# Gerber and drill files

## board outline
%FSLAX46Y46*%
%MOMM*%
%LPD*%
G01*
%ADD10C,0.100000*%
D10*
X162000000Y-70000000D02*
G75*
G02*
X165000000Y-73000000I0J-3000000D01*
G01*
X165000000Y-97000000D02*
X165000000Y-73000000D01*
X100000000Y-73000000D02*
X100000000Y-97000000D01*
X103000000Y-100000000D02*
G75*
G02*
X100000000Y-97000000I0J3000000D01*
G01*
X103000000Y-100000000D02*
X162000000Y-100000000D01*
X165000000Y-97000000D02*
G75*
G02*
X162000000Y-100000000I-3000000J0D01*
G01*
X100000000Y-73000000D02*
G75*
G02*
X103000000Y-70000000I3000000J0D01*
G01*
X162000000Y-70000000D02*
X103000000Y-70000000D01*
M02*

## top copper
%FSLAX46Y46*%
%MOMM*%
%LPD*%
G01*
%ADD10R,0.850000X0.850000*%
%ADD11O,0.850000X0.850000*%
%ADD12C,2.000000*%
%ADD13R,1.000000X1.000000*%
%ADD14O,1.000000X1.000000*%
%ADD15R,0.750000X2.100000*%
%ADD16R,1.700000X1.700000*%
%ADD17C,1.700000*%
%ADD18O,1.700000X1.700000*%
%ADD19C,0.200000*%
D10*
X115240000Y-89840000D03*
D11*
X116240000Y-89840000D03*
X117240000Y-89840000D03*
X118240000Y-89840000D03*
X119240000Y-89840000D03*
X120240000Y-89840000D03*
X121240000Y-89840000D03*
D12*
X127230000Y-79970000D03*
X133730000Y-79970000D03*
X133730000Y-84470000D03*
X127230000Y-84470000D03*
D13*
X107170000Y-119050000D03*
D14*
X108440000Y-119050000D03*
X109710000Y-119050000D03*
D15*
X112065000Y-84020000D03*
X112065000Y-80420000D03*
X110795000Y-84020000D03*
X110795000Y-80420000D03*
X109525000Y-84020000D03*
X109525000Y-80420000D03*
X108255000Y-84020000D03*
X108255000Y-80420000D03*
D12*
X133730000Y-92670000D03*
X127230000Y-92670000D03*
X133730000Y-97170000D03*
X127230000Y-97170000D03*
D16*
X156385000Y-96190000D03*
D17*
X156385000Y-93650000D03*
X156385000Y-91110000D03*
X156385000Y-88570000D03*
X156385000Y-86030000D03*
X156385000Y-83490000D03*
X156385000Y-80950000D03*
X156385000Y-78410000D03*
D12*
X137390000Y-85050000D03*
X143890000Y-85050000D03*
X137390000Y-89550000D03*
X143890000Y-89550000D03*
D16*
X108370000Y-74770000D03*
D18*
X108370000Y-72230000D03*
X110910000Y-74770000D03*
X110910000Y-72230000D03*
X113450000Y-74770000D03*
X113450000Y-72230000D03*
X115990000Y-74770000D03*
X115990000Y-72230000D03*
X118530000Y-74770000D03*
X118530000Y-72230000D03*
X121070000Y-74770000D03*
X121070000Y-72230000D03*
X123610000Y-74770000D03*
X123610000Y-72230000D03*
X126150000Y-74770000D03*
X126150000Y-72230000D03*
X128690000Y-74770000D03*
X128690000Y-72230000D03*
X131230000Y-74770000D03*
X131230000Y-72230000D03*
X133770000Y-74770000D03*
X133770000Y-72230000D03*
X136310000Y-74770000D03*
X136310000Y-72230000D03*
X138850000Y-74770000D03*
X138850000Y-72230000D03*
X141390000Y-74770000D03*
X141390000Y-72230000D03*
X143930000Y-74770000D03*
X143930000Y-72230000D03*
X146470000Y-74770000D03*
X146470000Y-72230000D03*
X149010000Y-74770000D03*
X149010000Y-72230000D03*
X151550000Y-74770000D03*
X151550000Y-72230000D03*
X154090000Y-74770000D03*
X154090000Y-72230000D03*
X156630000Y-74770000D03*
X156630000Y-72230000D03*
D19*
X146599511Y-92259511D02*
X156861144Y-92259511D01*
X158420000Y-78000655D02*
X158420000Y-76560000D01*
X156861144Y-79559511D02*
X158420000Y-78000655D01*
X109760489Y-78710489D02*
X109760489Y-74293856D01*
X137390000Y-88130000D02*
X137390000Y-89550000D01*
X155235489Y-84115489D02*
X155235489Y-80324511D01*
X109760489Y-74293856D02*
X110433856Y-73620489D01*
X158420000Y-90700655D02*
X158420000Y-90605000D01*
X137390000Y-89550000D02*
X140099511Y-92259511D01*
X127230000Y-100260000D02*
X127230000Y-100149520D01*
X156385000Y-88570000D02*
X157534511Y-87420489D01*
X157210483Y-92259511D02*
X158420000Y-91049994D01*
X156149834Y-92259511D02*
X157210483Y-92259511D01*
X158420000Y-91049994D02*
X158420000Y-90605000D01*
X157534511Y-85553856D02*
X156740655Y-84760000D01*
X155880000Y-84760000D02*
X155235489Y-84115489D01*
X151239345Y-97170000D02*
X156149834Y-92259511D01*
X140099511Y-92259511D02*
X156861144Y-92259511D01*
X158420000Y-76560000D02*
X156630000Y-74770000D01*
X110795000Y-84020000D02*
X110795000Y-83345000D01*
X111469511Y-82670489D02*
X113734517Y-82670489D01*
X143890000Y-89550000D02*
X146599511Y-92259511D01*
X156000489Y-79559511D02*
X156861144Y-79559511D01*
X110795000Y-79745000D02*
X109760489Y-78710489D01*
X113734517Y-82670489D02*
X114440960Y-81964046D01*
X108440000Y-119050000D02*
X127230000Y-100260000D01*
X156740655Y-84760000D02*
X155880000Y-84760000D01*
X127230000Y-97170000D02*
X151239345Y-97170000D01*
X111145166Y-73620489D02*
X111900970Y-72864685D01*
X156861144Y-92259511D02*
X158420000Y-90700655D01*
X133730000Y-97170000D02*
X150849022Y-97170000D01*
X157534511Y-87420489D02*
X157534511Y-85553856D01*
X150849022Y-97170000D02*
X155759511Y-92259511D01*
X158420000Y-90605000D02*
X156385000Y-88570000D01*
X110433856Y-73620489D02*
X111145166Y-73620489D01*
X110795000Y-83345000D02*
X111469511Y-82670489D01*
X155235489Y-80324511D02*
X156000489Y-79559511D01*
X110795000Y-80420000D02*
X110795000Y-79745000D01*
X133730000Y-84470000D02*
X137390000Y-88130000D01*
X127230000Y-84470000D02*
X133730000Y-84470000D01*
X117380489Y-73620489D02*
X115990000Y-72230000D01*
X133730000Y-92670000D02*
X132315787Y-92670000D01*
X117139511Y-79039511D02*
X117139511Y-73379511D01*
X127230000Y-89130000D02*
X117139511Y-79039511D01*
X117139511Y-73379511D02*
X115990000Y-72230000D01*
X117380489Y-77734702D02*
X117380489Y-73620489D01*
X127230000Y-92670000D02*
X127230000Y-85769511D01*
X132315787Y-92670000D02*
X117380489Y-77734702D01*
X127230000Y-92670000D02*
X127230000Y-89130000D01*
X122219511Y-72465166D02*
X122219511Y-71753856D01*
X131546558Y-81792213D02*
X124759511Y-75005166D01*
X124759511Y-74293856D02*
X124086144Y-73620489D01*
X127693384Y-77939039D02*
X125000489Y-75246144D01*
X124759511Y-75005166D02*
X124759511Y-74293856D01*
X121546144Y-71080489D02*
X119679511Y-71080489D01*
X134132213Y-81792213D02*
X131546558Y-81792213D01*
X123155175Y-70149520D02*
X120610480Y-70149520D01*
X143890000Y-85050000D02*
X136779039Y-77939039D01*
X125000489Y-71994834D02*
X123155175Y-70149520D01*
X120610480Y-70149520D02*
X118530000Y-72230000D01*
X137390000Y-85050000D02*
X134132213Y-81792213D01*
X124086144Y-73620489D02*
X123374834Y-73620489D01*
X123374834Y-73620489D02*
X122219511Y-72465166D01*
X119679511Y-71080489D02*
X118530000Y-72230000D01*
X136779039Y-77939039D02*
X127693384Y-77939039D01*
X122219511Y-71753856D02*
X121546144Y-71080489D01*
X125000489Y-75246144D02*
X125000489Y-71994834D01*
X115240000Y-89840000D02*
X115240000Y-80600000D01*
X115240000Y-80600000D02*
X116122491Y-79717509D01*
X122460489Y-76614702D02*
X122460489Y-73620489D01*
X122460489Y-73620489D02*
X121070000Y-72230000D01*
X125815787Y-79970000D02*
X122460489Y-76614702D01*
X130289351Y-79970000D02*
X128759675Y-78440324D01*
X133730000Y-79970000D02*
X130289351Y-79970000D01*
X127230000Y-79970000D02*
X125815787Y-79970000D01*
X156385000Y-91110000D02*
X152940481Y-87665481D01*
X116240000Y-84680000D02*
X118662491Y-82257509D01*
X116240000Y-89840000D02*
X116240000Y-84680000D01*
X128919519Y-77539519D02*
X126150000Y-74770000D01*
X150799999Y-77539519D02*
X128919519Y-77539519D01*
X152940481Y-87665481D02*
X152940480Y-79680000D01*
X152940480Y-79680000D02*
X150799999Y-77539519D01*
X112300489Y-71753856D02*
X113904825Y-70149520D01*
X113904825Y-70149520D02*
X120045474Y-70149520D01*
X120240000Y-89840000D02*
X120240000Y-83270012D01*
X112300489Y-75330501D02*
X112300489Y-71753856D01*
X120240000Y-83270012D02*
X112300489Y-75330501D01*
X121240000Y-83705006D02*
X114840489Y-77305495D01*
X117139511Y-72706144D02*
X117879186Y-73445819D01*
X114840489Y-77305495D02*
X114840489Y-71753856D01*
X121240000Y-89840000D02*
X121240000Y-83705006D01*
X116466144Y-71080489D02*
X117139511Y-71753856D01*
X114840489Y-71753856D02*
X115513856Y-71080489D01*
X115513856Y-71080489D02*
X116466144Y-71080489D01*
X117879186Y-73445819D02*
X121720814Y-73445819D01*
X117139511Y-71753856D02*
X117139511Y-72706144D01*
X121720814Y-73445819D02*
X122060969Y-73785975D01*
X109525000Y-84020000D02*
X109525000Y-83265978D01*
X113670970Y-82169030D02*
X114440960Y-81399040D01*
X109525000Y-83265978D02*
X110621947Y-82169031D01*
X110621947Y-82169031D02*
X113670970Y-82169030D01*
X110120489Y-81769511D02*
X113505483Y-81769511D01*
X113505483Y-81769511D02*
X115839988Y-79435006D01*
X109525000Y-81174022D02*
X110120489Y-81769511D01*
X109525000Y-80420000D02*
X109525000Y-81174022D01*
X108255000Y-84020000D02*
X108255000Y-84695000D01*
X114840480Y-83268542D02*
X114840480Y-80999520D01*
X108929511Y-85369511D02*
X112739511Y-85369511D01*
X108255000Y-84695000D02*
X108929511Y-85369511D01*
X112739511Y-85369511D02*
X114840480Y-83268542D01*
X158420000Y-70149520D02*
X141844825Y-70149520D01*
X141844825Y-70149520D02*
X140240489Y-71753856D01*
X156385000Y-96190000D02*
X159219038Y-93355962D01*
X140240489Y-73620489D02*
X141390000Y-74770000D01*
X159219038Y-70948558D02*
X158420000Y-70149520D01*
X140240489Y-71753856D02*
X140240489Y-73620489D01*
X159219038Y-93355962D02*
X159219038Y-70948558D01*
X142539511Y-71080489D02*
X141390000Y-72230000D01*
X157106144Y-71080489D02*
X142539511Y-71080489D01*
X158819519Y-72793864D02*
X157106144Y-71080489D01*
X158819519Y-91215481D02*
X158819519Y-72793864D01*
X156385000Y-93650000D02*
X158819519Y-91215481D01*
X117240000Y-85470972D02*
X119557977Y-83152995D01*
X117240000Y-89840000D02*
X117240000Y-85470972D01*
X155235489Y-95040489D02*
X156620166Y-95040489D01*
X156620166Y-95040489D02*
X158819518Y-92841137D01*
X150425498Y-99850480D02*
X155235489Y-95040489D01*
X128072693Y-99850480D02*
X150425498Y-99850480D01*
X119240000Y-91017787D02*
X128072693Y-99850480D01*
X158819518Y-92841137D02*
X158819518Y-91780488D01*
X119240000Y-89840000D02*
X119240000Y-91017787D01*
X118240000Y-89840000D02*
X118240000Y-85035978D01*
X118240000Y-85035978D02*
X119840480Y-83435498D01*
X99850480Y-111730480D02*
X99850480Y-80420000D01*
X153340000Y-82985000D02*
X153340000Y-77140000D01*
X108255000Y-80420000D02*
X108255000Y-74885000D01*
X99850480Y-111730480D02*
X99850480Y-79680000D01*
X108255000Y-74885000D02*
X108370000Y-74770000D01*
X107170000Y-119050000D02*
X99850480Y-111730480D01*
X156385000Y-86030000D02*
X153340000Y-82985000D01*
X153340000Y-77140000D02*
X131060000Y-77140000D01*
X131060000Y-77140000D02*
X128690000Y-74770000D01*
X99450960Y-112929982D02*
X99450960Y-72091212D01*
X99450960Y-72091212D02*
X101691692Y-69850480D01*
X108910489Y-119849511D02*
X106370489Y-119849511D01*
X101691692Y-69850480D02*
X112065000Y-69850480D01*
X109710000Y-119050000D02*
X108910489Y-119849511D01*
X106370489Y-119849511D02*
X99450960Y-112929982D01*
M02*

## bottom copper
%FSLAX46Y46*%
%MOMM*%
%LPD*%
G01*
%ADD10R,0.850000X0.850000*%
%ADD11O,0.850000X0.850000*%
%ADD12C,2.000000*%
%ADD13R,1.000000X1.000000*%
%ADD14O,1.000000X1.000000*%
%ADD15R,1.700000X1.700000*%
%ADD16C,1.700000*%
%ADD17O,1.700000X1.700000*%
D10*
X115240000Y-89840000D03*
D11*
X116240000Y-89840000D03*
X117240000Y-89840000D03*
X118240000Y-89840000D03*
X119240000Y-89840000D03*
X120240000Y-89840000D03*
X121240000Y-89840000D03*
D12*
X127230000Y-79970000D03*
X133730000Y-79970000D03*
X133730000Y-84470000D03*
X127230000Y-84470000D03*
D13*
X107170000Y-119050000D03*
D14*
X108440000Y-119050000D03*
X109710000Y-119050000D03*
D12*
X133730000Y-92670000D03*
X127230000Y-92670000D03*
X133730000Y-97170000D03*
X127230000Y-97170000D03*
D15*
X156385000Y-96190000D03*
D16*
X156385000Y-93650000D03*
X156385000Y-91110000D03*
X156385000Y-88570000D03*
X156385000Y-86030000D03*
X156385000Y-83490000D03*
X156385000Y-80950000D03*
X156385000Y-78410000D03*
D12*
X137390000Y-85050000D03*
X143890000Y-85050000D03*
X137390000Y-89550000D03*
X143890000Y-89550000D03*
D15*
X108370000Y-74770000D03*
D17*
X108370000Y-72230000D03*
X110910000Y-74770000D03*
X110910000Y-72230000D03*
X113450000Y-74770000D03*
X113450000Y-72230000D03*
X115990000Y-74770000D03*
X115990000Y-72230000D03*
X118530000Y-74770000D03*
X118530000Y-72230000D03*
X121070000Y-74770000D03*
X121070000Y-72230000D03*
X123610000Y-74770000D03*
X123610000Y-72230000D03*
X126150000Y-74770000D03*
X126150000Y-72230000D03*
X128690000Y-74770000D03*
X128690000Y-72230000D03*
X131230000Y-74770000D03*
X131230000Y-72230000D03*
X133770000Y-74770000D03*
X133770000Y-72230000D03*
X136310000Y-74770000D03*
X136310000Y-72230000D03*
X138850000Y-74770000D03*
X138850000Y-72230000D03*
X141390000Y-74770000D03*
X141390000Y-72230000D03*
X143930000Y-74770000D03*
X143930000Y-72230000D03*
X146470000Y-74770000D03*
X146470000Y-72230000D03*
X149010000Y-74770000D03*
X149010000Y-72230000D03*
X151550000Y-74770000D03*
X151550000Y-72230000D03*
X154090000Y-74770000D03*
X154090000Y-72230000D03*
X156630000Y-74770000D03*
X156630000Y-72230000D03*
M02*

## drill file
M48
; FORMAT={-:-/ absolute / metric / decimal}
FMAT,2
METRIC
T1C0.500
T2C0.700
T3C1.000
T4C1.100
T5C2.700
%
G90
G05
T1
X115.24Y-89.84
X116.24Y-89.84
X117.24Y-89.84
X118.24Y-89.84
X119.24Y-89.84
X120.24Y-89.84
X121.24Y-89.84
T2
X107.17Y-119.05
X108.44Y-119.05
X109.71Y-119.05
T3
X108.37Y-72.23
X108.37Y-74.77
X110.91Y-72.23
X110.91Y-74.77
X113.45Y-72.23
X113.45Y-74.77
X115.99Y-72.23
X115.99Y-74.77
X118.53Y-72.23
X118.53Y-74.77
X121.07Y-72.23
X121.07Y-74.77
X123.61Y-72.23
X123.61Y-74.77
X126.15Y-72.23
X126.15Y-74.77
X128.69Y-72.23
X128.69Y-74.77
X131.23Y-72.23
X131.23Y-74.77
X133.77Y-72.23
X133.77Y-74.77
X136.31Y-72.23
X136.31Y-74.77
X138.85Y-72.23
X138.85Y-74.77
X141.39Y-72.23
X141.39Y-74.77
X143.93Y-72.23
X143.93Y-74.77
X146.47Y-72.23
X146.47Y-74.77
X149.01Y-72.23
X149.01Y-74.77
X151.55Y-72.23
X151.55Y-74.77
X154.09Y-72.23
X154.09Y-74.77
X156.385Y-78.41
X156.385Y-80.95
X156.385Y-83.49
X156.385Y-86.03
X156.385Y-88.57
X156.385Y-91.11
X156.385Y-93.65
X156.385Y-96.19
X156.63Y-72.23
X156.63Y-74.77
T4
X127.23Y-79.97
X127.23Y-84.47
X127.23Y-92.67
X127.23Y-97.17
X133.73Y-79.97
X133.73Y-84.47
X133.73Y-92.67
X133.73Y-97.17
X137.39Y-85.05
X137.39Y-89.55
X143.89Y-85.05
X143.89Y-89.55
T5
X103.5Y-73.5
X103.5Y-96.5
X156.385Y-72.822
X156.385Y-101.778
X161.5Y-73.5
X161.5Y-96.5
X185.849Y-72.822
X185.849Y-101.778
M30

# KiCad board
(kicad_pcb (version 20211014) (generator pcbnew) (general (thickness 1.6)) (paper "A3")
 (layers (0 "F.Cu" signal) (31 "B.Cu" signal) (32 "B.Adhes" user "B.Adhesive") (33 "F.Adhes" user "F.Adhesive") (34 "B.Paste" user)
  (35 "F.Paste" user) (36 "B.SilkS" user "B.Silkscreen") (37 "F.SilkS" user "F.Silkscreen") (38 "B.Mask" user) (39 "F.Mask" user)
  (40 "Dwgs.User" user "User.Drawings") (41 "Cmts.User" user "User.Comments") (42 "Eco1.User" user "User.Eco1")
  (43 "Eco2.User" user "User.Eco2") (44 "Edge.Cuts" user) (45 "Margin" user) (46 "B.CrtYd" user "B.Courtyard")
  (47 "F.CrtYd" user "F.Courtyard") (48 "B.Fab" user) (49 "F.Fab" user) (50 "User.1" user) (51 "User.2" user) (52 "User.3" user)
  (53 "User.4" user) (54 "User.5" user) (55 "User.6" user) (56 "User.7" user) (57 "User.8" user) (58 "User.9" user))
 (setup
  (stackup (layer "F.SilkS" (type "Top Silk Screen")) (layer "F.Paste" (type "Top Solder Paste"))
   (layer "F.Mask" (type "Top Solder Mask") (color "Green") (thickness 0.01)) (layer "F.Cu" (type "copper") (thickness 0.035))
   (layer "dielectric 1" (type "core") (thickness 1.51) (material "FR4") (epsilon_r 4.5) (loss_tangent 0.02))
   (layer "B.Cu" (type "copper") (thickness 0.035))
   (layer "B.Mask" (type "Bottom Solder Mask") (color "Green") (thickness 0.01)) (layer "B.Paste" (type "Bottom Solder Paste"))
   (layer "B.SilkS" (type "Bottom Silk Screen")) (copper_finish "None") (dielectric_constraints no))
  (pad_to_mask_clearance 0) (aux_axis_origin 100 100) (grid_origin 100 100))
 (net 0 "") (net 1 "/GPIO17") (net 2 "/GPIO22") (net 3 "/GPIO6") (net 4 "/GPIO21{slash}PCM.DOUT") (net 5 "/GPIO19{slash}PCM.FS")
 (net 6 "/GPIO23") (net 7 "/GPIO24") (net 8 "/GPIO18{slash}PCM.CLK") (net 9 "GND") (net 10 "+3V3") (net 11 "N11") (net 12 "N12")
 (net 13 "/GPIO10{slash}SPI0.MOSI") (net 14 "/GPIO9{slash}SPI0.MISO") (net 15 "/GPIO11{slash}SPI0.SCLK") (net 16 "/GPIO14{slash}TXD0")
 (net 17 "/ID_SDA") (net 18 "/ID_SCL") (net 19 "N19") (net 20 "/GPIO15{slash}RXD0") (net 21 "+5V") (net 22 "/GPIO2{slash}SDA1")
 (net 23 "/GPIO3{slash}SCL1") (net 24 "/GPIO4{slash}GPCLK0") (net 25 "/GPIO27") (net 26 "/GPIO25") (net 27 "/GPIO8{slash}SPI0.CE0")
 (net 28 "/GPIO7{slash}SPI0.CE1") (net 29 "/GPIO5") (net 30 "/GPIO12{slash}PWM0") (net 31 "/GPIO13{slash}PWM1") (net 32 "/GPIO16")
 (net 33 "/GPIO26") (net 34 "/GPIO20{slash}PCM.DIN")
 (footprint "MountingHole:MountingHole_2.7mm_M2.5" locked (layer "F.Cu") (at 161.5 73.5)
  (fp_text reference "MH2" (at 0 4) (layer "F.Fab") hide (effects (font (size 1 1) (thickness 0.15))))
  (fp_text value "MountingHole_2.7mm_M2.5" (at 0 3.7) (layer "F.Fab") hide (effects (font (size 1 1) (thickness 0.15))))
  (pad "" np_thru_hole circle locked (at 0 0) (size 2.7 2.7) (drill 2.7) (layers *.Cu *.Mask)))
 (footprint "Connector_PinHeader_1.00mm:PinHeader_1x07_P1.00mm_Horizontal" (layer "F.Cu") (at 115.24 89.84 90)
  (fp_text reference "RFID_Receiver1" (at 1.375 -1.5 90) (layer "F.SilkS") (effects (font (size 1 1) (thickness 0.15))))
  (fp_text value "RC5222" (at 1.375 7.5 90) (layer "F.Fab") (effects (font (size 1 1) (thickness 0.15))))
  (pad "1" thru_hole rect (at 0 0 90) (size 0.85 0.85) (drill 0.5) (layers *.Cu *.Mask) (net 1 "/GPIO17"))
  (pad "2" thru_hole oval (at 0 1 90) (size 0.85 0.85) (drill 0.5) (layers *.Cu *.Mask) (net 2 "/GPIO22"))
  (pad "3" thru_hole oval (at 0 2 90) (size 0.85 0.85) (drill 0.5) (layers *.Cu *.Mask) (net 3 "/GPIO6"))
  (pad "4" thru_hole oval (at 0 3 90) (size 0.85 0.85) (drill 0.5) (layers *.Cu *.Mask) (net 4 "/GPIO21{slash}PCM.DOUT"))
  (pad "5" thru_hole oval (at 0 4 90) (size 0.85 0.85) (drill 0.5) (layers *.Cu *.Mask) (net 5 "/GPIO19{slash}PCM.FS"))
  (pad "6" thru_hole oval (at 0 5 90) (size 0.85 0.85) (drill 0.5) (layers *.Cu *.Mask) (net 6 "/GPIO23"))
  (pad "7" thru_hole oval (at 0 6 90) (size 0.85 0.85) (drill 0.5) (layers *.Cu *.Mask) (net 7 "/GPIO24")))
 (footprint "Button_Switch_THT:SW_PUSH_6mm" (layer "F.Cu") (at 127.23 79.97)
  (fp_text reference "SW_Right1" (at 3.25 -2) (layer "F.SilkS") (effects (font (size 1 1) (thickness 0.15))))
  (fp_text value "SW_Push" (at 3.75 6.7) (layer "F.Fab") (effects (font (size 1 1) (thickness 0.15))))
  (pad "1" thru_hole circle (at 0 0 90) (size 2 2) (drill 1.1) (layers *.Cu *.Mask) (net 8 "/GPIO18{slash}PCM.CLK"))
  (pad "1" thru_hole circle (at 6.5 0 90) (size 2 2) (drill 1.1) (layers *.Cu *.Mask) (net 8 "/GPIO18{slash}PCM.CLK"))
  (pad "2" thru_hole circle (at 6.5 4.5 90) (size 2 2) (drill 1.1) (layers *.Cu *.Mask) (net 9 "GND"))
  (pad "2" thru_hole circle (at 0 4.5 90) (size 2 2) (drill 1.1) (layers *.Cu *.Mask) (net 9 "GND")))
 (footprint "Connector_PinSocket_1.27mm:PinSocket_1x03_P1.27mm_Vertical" (layer "F.Cu") (at 107.17 119.05 90)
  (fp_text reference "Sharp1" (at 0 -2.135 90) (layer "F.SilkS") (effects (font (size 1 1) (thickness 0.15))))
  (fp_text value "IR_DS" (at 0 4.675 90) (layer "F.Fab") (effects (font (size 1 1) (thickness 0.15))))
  (pad "1" thru_hole rect (at 0 0 90) (size 1 1) (drill 0.7) (layers *.Cu *.Mask) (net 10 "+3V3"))
  (pad "2" thru_hole oval (at 0 1.27 90) (size 1 1) (drill 0.7) (layers *.Cu *.Mask) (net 9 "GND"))
  (pad "3" thru_hole oval (at 0 2.54 90) (size 1 1) (drill 0.7) (layers *.Cu *.Mask) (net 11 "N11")))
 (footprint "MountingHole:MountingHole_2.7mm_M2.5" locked (layer "F.Cu") (at 103.5 96.5)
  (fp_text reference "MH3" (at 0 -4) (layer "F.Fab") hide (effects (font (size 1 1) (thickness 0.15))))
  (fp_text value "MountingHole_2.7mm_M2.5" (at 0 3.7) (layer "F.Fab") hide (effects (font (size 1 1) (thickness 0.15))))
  (pad "" np_thru_hole circle locked (at 0 0) (size 2.7 2.7) (drill 2.7) (layers *.Cu *.Mask)))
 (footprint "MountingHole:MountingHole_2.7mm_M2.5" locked (layer "F.Cu") (at 103.5 73.5)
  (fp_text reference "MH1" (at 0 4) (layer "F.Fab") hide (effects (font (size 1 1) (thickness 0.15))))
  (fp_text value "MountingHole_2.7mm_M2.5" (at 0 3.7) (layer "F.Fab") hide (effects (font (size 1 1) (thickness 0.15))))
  (pad "" np_thru_hole circle locked (at 0 0) (size 2.7 2.7) (drill 2.7) (layers *.Cu *.Mask)))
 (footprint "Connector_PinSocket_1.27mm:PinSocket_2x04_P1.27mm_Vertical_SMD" (layer "F.Cu") (at 110.16 82.22 -90)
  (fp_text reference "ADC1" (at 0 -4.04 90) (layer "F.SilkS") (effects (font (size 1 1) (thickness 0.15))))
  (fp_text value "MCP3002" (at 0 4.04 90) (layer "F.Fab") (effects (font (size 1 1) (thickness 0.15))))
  (pad "1" smd rect (at 1.8 -1.905 270) (size 2.1 0.75) (layers "F.Cu" "F.Paste" "F.Mask") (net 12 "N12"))
  (pad "2" smd rect (at -1.8 -1.905 270) (size 2.1 0.75) (layers "F.Cu" "F.Paste" "F.Mask") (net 11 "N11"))
  (pad "3" smd rect (at 1.8 -0.635 270) (size 2.1 0.75) (layers "F.Cu" "F.Paste" "F.Mask") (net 9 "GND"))
  (pad "4" smd rect (at -1.8 -0.635 270) (size 2.1 0.75) (layers "F.Cu" "F.Paste" "F.Mask") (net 9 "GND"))
  (pad "5" smd rect (at 1.8 0.635 270) (size 2.1 0.75) (layers "F.Cu" "F.Paste" "F.Mask") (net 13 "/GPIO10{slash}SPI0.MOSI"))
  (pad "6" smd rect (at -1.8 0.635 270) (size 2.1 0.75) (layers "F.Cu" "F.Paste" "F.Mask") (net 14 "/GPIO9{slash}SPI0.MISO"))
  (pad "7" smd rect (at 1.8 1.905 270) (size 2.1 0.75) (layers "F.Cu" "F.Paste" "F.Mask") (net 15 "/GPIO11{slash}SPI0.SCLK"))
  (pad "8" smd rect (at -1.8 1.905 270) (size 2.1 0.75) (layers "F.Cu" "F.Paste" "F.Mask") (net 10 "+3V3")))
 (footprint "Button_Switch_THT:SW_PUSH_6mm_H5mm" (layer "F.Cu") (at 127.23 92.67)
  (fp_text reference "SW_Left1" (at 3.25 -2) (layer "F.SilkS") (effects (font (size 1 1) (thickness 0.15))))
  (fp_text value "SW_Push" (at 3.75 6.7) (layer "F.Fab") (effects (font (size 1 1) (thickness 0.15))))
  (pad "1" thru_hole circle (at 6.5 0 90) (size 2 2) (drill 1.1) (layers *.Cu *.Mask) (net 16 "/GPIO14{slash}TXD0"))
  (pad "1" thru_hole circle (at 0 0 90) (size 2 2) (drill 1.1) (layers *.Cu *.Mask) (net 16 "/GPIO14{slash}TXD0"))
  (pad "2" thru_hole circle (at 6.5 4.5 90) (size 2 2) (drill 1.1) (layers *.Cu *.Mask) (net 9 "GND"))
  (pad "2" thru_hole circle (at 0 4.5 90) (size 2 2) (drill 1.1) (layers *.Cu *.Mask) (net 9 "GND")))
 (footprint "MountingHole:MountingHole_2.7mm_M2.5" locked (layer "F.Cu") (at 161.5 96.5)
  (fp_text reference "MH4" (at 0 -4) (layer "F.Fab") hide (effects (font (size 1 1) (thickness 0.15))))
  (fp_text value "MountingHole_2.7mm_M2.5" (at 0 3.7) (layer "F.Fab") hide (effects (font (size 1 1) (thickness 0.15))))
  (pad "" np_thru_hole circle locked (at 0 0) (size 2.7 2.7) (drill 2.7) (layers *.Cu *.Mask)))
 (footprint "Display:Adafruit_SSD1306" (layer "F.Cu") (at 156.385 96.19 90)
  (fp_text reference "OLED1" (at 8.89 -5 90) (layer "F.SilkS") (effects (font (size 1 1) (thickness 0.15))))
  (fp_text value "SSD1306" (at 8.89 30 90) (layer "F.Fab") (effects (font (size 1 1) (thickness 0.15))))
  (pad "" np_thru_hole circle (at -5.588 29.464 90) (size 2.7 2.7) (drill 2.7) (layers *.Cu *.Mask))
  (pad "" np_thru_hole circle (at 23.368 29.464 90) (size 2.7 2.7) (drill 2.7) (layers *.Cu *.Mask))
  (pad "" np_thru_hole circle (at 23.368 0 90) (size 2.7 2.7) (drill 2.7) (layers *.Cu *.Mask))
  (pad "" np_thru_hole circle (at -5.588 0 90) (size 2.7 2.7) (drill 2.7) (layers *.Cu *.Mask))
  (pad "1" thru_hole rect (at 0 0 90) (size 1.7 1.7) (drill 1) (layers *.Cu *.Mask) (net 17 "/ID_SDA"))
  (pad "2" thru_hole circle (at 2.54 0 90) (size 1.7 1.7) (drill 1) (layers *.Cu *.Mask) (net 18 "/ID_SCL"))
  (pad "3" thru_hole circle (at 5.08 0 90) (size 1.7 1.7) (drill 1) (layers *.Cu *.Mask) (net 2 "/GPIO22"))
  (pad "4" thru_hole circle (at 7.62 0 90) (size 1.7 1.7) (drill 1) (layers *.Cu *.Mask) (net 9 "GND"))
  (pad "5" thru_hole circle (at 10.16 0 90) (size 1.7 1.7) (drill 1) (layers *.Cu *.Mask) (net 10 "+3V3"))
  (pad "6" thru_hole circle (at 12.7 0 90) (size 1.7 1.7) (drill 1) (layers *.Cu *.Mask) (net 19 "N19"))
  (pad "7" thru_hole circle (at 15.24 0 90) (size 1.7 1.7) (drill 1) (layers *.Cu *.Mask))
  (pad "8" thru_hole circle (at 17.78 0 90) (size 1.7 1.7) (drill 1) (layers *.Cu *.Mask)))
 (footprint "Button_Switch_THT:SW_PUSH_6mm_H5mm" (layer "F.Cu") (at 137.39 85.05)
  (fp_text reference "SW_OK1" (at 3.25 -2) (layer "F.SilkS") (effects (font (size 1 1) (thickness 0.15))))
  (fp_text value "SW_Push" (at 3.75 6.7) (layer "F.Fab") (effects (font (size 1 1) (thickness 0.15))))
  (pad "1" thru_hole circle (at 0 0 90) (size 2 2) (drill 1.1) (layers *.Cu *.Mask) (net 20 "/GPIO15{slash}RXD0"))
  (pad "1" thru_hole circle (at 6.5 0 90) (size 2 2) (drill 1.1) (layers *.Cu *.Mask) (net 20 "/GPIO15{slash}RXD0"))
  (pad "2" thru_hole circle (at 0 4.5 90) (size 2 2) (drill 1.1) (layers *.Cu *.Mask) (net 9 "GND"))
  (pad "2" thru_hole circle (at 6.5 4.5 90) (size 2 2) (drill 1.1) (layers *.Cu *.Mask) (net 9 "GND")))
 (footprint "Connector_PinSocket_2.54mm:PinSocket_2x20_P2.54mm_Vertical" (layer "B.Cu") (at 108.37 74.77 -90)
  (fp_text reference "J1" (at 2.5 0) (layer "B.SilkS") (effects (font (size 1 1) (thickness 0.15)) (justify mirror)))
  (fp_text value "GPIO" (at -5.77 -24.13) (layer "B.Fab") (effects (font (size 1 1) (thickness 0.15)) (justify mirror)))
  (pad "1" thru_hole rect locked (at 0 0 270) (size 1.7 1.7) (drill 1) (layers *.Cu *.Mask) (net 10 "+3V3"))
  (pad "2" thru_hole oval locked (at -2.54 0 270) (size 1.7 1.7) (drill 1) (layers *.Cu *.Mask) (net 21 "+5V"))
  (pad "3" thru_hole oval locked (at 0 -2.54 270) (size 1.7 1.7) (drill 1) (layers *.Cu *.Mask) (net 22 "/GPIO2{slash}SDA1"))
  (pad "4" thru_hole oval locked (at -2.54 -2.54 270) (size 1.7 1.7) (drill 1) (layers *.Cu *.Mask) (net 21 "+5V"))
  (pad "5" thru_hole oval locked (at 0 -5.08 270) (size 1.7 1.7) (drill 1) (layers *.Cu *.Mask) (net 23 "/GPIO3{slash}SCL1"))
  (pad "6" thru_hole oval locked (at -2.54 -5.08 270) (size 1.7 1.7) (drill 1) (layers *.Cu *.Mask) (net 9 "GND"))
  (pad "7" thru_hole oval locked (at 0 -7.62 270) (size 1.7 1.7) (drill 1) (layers *.Cu *.Mask) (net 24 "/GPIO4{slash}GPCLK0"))
  (pad "8" thru_hole oval locked (at -2.54 -7.62 270) (size 1.7 1.7) (drill 1) (layers *.Cu *.Mask) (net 16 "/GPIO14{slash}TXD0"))
  (pad "9" thru_hole oval locked (at 0 -10.16 270) (size 1.7 1.7) (drill 1) (layers *.Cu *.Mask) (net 9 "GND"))
  (pad "10" thru_hole oval locked (at -2.54 -10.16 270) (size 1.7 1.7) (drill 1) (layers *.Cu *.Mask) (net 20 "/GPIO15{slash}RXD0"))
  (pad "11" thru_hole oval locked (at 0 -12.7 270) (size 1.7 1.7) (drill 1) (layers *.Cu *.Mask) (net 1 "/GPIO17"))
  (pad "12" thru_hole oval locked (at -2.54 -12.7 270) (size 1.7 1.7) (drill 1) (layers *.Cu *.Mask) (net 8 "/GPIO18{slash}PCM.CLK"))
  (pad "13" thru_hole oval locked (at 0 -15.24 270) (size 1.7 1.7) (drill 1) (layers *.Cu *.Mask) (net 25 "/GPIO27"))
  (pad "14" thru_hole oval locked (at -2.54 -15.24 270) (size 1.7 1.7) (drill 1) (layers *.Cu *.Mask) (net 9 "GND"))
  (pad "15" thru_hole oval locked (at 0 -17.78 270) (size 1.7 1.7) (drill 1) (layers *.Cu *.Mask) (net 2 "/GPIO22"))
  (pad "16" thru_hole oval locked (at -2.54 -17.78 270) (size 1.7 1.7) (drill 1) (layers *.Cu *.Mask) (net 6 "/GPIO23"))
  (pad "17" thru_hole oval locked (at 0 -20.32 270) (size 1.7 1.7) (drill 1) (layers *.Cu *.Mask) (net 10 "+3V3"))
  (pad "18" thru_hole oval locked (at -2.54 -20.32 270) (size 1.7 1.7) (drill 1) (layers *.Cu *.Mask) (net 7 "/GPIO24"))
  (pad "19" thru_hole oval locked (at 0 -22.86 270) (size 1.7 1.7) (drill 1) (layers *.Cu *.Mask) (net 13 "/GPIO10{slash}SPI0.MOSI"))
  (pad "20" thru_hole oval locked (at -2.54 -22.86 270) (size 1.7 1.7) (drill 1) (layers *.Cu *.Mask) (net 9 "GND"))
  (pad "21" thru_hole oval locked (at 0 -25.4 270) (size 1.7 1.7) (drill 1) (layers *.Cu *.Mask) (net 14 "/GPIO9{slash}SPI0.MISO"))
  (pad "22" thru_hole oval locked (at -2.54 -25.4 270) (size 1.7 1.7) (drill 1) (layers *.Cu *.Mask) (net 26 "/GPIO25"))
  (pad "23" thru_hole oval locked (at 0 -27.94 270) (size 1.7 1.7) (drill 1) (layers *.Cu *.Mask) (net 15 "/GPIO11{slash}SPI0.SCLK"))
  (pad "24" thru_hole oval locked (at -2.54 -27.94 270) (size 1.7 1.7) (drill 1) (layers *.Cu *.Mask) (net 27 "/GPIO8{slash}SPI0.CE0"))
  (pad "25" thru_hole oval locked (at 0 -30.48 270) (size 1.7 1.7) (drill 1) (layers *.Cu *.Mask) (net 9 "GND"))
  (pad "26" thru_hole oval locked (at -2.54 -30.48 270) (size 1.7 1.7) (drill 1) (layers *.Cu *.Mask) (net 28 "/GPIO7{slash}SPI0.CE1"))
  (pad "27" thru_hole oval locked (at 0 -33.02 270) (size 1.7 1.7) (drill 1) (layers *.Cu *.Mask) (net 17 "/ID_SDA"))
  (pad "28" thru_hole oval locked (at -2.54 -33.02 270) (size 1.7 1.7) (drill 1) (layers *.Cu *.Mask) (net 18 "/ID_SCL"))
  (pad "29" thru_hole oval locked (at 0 -35.56 270) (size 1.7 1.7) (drill 1) (layers *.Cu *.Mask) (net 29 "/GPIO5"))
  (pad "30" thru_hole oval locked (at -2.54 -35.56 270) (size 1.7 1.7) (drill 1) (layers *.Cu *.Mask) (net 9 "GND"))
  (pad "31" thru_hole oval locked (at 0 -38.1 270) (size 1.7 1.7) (drill 1) (layers *.Cu *.Mask) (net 3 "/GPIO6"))
  (pad "32" thru_hole oval locked (at -2.54 -38.1 270) (size 1.7 1.7) (drill 1) (layers *.Cu *.Mask) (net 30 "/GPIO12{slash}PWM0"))
  (pad "33" thru_hole oval locked (at 0 -40.64 270) (size 1.7 1.7) (drill 1) (layers *.Cu *.Mask) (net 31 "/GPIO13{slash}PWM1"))
  (pad "34" thru_hole oval locked (at -2.54 -40.64 270) (size 1.7 1.7) (drill 1) (layers *.Cu *.Mask) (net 9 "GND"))
  (pad "35" thru_hole oval locked (at 0 -43.18 270) (size 1.7 1.7) (drill 1) (layers *.Cu *.Mask) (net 5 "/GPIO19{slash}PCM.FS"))
  (pad "36" thru_hole oval locked (at -2.54 -43.18 270) (size 1.7 1.7) (drill 1) (layers *.Cu *.Mask) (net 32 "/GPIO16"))
  (pad "37" thru_hole oval locked (at 0 -45.72 270) (size 1.7 1.7) (drill 1) (layers *.Cu *.Mask) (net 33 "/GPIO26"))
  (pad "38" thru_hole oval locked (at -2.54 -45.72 270) (size 1.7 1.7) (drill 1) (layers *.Cu *.Mask) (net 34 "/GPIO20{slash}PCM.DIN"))
  (pad "39" thru_hole oval locked (at 0 -48.26 270) (size 1.7 1.7) (drill 1) (layers *.Cu *.Mask) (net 9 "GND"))
  (pad "40" thru_hole oval locked (at -2.54 -48.26 270) (size 1.7 1.7) (drill 1) (layers *.Cu *.Mask) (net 4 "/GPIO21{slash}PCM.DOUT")))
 (gr_arc (start 162 70) (mid 164.12132 70.87868) (end 165 73) (layer "Edge.Cuts") (width 0.1))
 (gr_line (start 165 97) (end 165 73) (layer "Edge.Cuts") (width 0.1))
 (gr_line (start 100 73) (end 100 97) (layer "Edge.Cuts") (width 0.1))
 (gr_arc (start 103 100) (mid 100.87868 99.12132) (end 100 97) (layer "Edge.Cuts") (width 0.1))
 (gr_line (start 103 100) (end 162 100) (layer "Edge.Cuts") (width 0.1))
 (gr_arc (start 165 97) (mid 164.12132 99.12132) (end 162 100) (layer "Edge.Cuts") (width 0.1))
 (gr_arc (start 100 73) (mid 100.87868 70.87868) (end 103 70) (layer "Edge.Cuts") (width 0.1))
 (gr_line (start 162 70) (end 103 70) (layer "Edge.Cuts") (width 0.1))
 (segment (start 146.599511 92.259511) (end 156.861144 92.259511) (width 0.2) (layer "F.Cu") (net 9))
 (segment (start 158.42 78.000655) (end 158.42 76.56) (width 0.2) (layer "F.Cu") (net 9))
 (segment (start 156.861144 79.559511) (end 158.42 78.000655) (width 0.2) (layer "F.Cu") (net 9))
 (segment (start 109.760489 78.710489) (end 109.760489 74.293856) (width 0.2) (layer "F.Cu") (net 9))
 (segment (start 137.39 88.13) (end 137.39 89.55) (width 0.2) (layer "F.Cu") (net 9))
 (segment (start 155.235489 84.115489) (end 155.235489 80.324511) (width 0.2) (layer "F.Cu") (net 9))
 (segment (start 109.760489 74.293856) (end 110.433856 73.620489) (width 0.2) (layer "F.Cu") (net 9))
 (segment (start 158.42 90.700655) (end 158.42 90.605) (width 0.2) (layer "F.Cu") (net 9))
 (segment (start 137.39 89.55) (end 140.099511 92.259511) (width 0.2) (layer "F.Cu") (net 9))
 (segment (start 127.23 100.26) (end 127.23 100.14952) (width 0.2) (layer "F.Cu") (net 9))
 (segment (start 156.385 88.57) (end 157.534511 87.420489) (width 0.2) (layer "F.Cu") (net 9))
 (segment (start 157.210483 92.259511) (end 158.42 91.049994) (width 0.2) (layer "F.Cu") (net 9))
 (segment (start 156.149834 92.259511) (end 157.210483 92.259511) (width 0.2) (layer "F.Cu") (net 9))
 (segment (start 158.42 91.049994) (end 158.42 90.605) (width 0.2) (layer "F.Cu") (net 9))
 (segment (start 157.534511 85.553856) (end 156.740655 84.76) (width 0.2) (layer "F.Cu") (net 9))
 (segment (start 155.88 84.76) (end 155.235489 84.115489) (width 0.2) (layer "F.Cu") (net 9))
 (segment (start 151.239345 97.17) (end 156.149834 92.259511) (width 0.2) (layer "F.Cu") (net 9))
 (segment (start 140.099511 92.259511) (end 156.861144 92.259511) (width 0.2) (layer "F.Cu") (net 9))
 (segment (start 158.42 76.56) (end 156.63 74.77) (width 0.2) (layer "F.Cu") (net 9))
 (segment (start 110.795 84.02) (end 110.795 83.345) (width 0.2) (layer "F.Cu") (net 9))
 (segment (start 111.469511 82.670489) (end 113.734517 82.670489) (width 0.2) (layer "F.Cu") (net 9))
 (segment (start 143.89 89.55) (end 146.599511 92.259511) (width 0.2) (layer "F.Cu") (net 9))
 (segment (start 156.000489 79.559511) (end 156.861144 79.559511) (width 0.2) (layer "F.Cu") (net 9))
 (segment (start 110.795 79.745) (end 109.760489 78.710489) (width 0.2) (layer "F.Cu") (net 9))
 (segment (start 113.734517 82.670489) (end 114.44096 81.964046) (width 0.2) (layer "F.Cu") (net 9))
 (segment (start 108.44 119.05) (end 127.23 100.26) (width 0.2) (layer "F.Cu") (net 9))
 (segment (start 156.740655 84.76) (end 155.88 84.76) (width 0.2) (layer "F.Cu") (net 9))
 (segment (start 127.23 97.17) (end 151.239345 97.17) (width 0.2) (layer "F.Cu") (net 9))
 (segment (start 111.145166 73.620489) (end 111.90097 72.864685) (width 0.2) (layer "F.Cu") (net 9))
 (segment (start 156.861144 92.259511) (end 158.42 90.700655) (width 0.2) (layer "F.Cu") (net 9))
 (segment (start 133.73 97.17) (end 150.849022 97.17) (width 0.2) (layer "F.Cu") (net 9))
 (segment (start 157.534511 87.420489) (end 157.534511 85.553856) (width 0.2) (layer "F.Cu") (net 9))
 (segment (start 150.849022 97.17) (end 155.759511 92.259511) (width 0.2) (layer "F.Cu") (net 9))
 (segment (start 158.42 90.605) (end 156.385 88.57) (width 0.2) (layer "F.Cu") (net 9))
 (segment (start 110.433856 73.620489) (end 111.145166 73.620489) (width 0.2) (layer "F.Cu") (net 9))
 (segment (start 110.795 83.345) (end 111.469511 82.670489) (width 0.2) (layer "F.Cu") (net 9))
 (segment (start 155.235489 80.324511) (end 156.000489 79.559511) (width 0.2) (layer "F.Cu") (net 9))
 (segment (start 110.795 80.42) (end 110.795 79.745) (width 0.2) (layer "F.Cu") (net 9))
 (segment (start 133.73 84.47) (end 137.39 88.13) (width 0.2) (layer "F.Cu") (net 9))
 (segment (start 127.23 84.47) (end 133.73 84.47) (width 0.2) (layer "F.Cu") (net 9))
 (segment (start 117.380489 73.620489) (end 115.99 72.23) (width 0.2) (layer "F.Cu") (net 16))
 (segment (start 133.73 92.67) (end 132.315787 92.67) (width 0.2) (layer "F.Cu") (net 16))
 (segment (start 117.139511 79.039511) (end 117.139511 73.379511) (width 0.2) (layer "F.Cu") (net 16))
 (segment (start 127.23 89.13) (end 117.139511 79.039511) (width 0.2) (layer "F.Cu") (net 16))
 (segment (start 117.139511 73.379511) (end 115.99 72.23) (width 0.2) (layer "F.Cu") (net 16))
 (segment (start 117.380489 77.734702) (end 117.380489 73.620489) (width 0.2) (layer "F.Cu") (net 16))
 (segment (start 127.23 92.67) (end 127.23 85.769511) (width 0.2) (layer "F.Cu") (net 16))
 (segment (start 132.315787 92.67) (end 117.380489 77.734702) (width 0.2) (layer "F.Cu") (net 16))
 (segment (start 127.23 92.67) (end 127.23 89.13) (width 0.2) (layer "F.Cu") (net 16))
 (segment (start 122.219511 72.465166) (end 122.219511 71.753856) (width 0.2) (layer "F.Cu") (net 20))
 (segment (start 131.546558 81.792213) (end 124.759511 75.005166) (width 0.2) (layer "F.Cu") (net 20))
 (segment (start 124.759511 74.293856) (end 124.086144 73.620489) (width 0.2) (layer "F.Cu") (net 20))
 (segment (start 127.693384 77.939039) (end 125.000489 75.246144) (width 0.2) (layer "F.Cu") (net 20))
 (segment (start 124.759511 75.005166) (end 124.759511 74.293856) (width 0.2) (layer "F.Cu") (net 20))
 (segment (start 121.546144 71.080489) (end 119.679511 71.080489) (width 0.2) (layer "F.Cu") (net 20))
 (segment (start 134.132213 81.792213) (end 131.546558 81.792213) (width 0.2) (layer "F.Cu") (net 20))
 (segment (start 123.155175 70.14952) (end 120.61048 70.14952) (width 0.2) (layer "F.Cu") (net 20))
 (segment (start 143.89 85.05) (end 136.779039 77.939039) (width 0.2) (layer "F.Cu") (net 20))
 (segment (start 125.000489 71.994834) (end 123.155175 70.14952) (width 0.2) (layer "F.Cu") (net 20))
 (segment (start 120.61048 70.14952) (end 118.53 72.23) (width 0.2) (layer "F.Cu") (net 20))
 (segment (start 137.39 85.05) (end 134.132213 81.792213) (width 0.2) (layer "F.Cu") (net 20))
 (segment (start 124.086144 73.620489) (end 123.374834 73.620489) (width 0.2) (layer "F.Cu") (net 20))
 (segment (start 123.374834 73.620489) (end 122.219511 72.465166) (width 0.2) (layer "F.Cu") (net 20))
 (segment (start 119.679511 71.080489) (end 118.53 72.23) (width 0.2) (layer "F.Cu") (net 20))
 (segment (start 136.779039 77.939039) (end 127.693384 77.939039) (width 0.2) (layer "F.Cu") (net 20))
 (segment (start 122.219511 71.753856) (end 121.546144 71.080489) (width 0.2) (layer "F.Cu") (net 20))
 (segment (start 125.000489 75.246144) (end 125.000489 71.994834) (width 0.2) (layer "F.Cu") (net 20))
 (segment (start 115.24 89.84) (end 115.24 80.6) (width 0.2) (layer "F.Cu") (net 1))
 (segment (start 115.24 80.6) (end 116.122491 79.717509) (width 0.2) (layer "F.Cu") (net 1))
 (segment (start 122.460489 76.614702) (end 122.460489 73.620489) (width 0.2) (layer "F.Cu") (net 8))
 (segment (start 122.460489 73.620489) (end 121.07 72.23) (width 0.2) (layer "F.Cu") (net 8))
 (segment (start 125.815787 79.97) (end 122.460489 76.614702) (width 0.2) (layer "F.Cu") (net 8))
 (segment (start 130.289351 79.97) (end 128.759675 78.440324) (width 0.2) (layer "F.Cu") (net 8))
 (segment (start 133.73 79.97) (end 130.289351 79.97) (width 0.2) (layer "F.Cu") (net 8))
 (segment (start 127.23 79.97) (end 125.815787 79.97) (width 0.2) (layer "F.Cu") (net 8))
 (segment (start 156.385 91.11) (end 152.940481 87.665481) (width 0.2) (layer "F.Cu") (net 2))
 (segment (start 116.24 84.68) (end 118.662491 82.257509) (width 0.2) (layer "F.Cu") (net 2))
 (segment (start 116.24 89.84) (end 116.24 84.68) (width 0.2) (layer "F.Cu") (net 2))
 (segment (start 128.919519 77.539519) (end 126.15 74.77) (width 0.2) (layer "F.Cu") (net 2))
 (segment (start 150.799999 77.539519) (end 128.919519 77.539519) (width 0.2) (layer "F.Cu") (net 2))
 (segment (start 152.940481 87.665481) (end 152.94048 79.68) (width 0.2) (layer "F.Cu") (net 2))
 (segment (start 152.94048 79.68) (end 150.799999 77.539519) (width 0.2) (layer "F.Cu") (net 2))
 (segment (start 112.300489 71.753856) (end 113.904825 70.14952) (width 0.2) (layer "F.Cu") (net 6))
 (segment (start 113.904825 70.14952) (end 120.045474 70.14952) (width 0.2) (layer "F.Cu") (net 6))
 (segment (start 120.24 89.84) (end 120.24 83.270012) (width 0.2) (layer "F.Cu") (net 6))
 (segment (start 112.300489 75.330501) (end 112.300489 71.753856) (width 0.2) (layer "F.Cu") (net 6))
 (segment (start 120.24 83.270012) (end 112.300489 75.330501) (width 0.2) (layer "F.Cu") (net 6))
 (segment (start 121.24 83.705006) (end 114.840489 77.305495) (width 0.2) (layer "F.Cu") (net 7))
 (segment (start 117.139511 72.706144) (end 117.879186 73.445819) (width 0.2) (layer "F.Cu") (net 7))
 (segment (start 114.840489 77.305495) (end 114.840489 71.753856) (width 0.2) (layer "F.Cu") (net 7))
 (segment (start 121.24 89.84) (end 121.24 83.705006) (width 0.2) (layer "F.Cu") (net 7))
 (segment (start 116.466144 71.080489) (end 117.139511 71.753856) (width 0.2) (layer "F.Cu") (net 7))
 (segment (start 114.840489 71.753856) (end 115.513856 71.080489) (width 0.2) (layer "F.Cu") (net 7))
 (segment (start 115.513856 71.080489) (end 116.466144 71.080489) (width 0.2) (layer "F.Cu") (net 7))
 (segment (start 117.879186 73.445819) (end 121.720814 73.445819) (width 0.2) (layer "F.Cu") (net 7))
 (segment (start 117.139511 71.753856) (end 117.139511 72.706144) (width 0.2) (layer "F.Cu") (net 7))
 (segment (start 121.720814 73.445819) (end 122.060969 73.785975) (width 0.2) (layer "F.Cu") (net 7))
 (segment (start 109.525 84.02) (end 109.525 83.265978) (width 0.2) (layer "F.Cu") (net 13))
 (segment (start 113.67097 82.16903) (end 114.44096 81.39904) (width 0.2) (layer "F.Cu") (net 13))
 (segment (start 109.525 83.265978) (end 110.621947 82.169031) (width 0.2) (layer "F.Cu") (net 13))
 (segment (start 110.621947 82.169031) (end 113.67097 82.16903) (width 0.2) (layer "F.Cu") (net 13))
 (segment (start 110.120489 81.769511) (end 113.505483 81.769511) (width 0.2) (layer "F.Cu") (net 14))
 (segment (start 113.505483 81.769511) (end 115.839988 79.435006) (width 0.2) (layer "F.Cu") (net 14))
 (segment (start 109.525 81.174022) (end 110.120489 81.769511) (width 0.2) (layer "F.Cu") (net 14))
 (segment (start 109.525 80.42) (end 109.525 81.174022) (width 0.2) (layer "F.Cu") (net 14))
 (segment (start 108.255 84.02) (end 108.255 84.695) (width 0.2) (layer "F.Cu") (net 15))
 (segment (start 114.84048 83.268542) (end 114.84048 80.99952) (width 0.2) (layer "F.Cu") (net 15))
 (segment (start 108.929511 85.369511) (end 112.739511 85.369511) (width 0.2) (layer "F.Cu") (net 15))
 (segment (start 108.255 84.695) (end 108.929511 85.369511) (width 0.2) (layer "F.Cu") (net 15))
 (segment (start 112.739511 85.369511) (end 114.84048 83.268542) (width 0.2) (layer "F.Cu") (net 15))
 (segment (start 158.42 70.14952) (end 141.844825 70.14952) (width 0.2) (layer "F.Cu") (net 17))
 (segment (start 141.844825 70.14952) (end 140.240489 71.753856) (width 0.2) (layer "F.Cu") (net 17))
 (segment (start 156.385 96.19) (end 159.219038 93.355962) (width 0.2) (layer "F.Cu") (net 17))
 (segment (start 140.240489 73.620489) (end 141.39 74.77) (width 0.2) (layer "F.Cu") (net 17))
 (segment (start 159.219038 70.948558) (end 158.42 70.14952) (width 0.2) (layer "F.Cu") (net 17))
 (segment (start 140.240489 71.753856) (end 140.240489 73.620489) (width 0.2) (layer "F.Cu") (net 17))
 (segment (start 159.219038 93.355962) (end 159.219038 70.948558) (width 0.2) (layer "F.Cu") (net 17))
 (segment (start 142.539511 71.080489) (end 141.39 72.23) (width 0.2) (layer "F.Cu") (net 18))
 (segment (start 157.106144 71.080489) (end 142.539511 71.080489) (width 0.2) (layer "F.Cu") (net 18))
 (segment (start 158.819519 72.793864) (end 157.106144 71.080489) (width 0.2) (layer "F.Cu") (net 18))
 (segment (start 158.819519 91.215481) (end 158.819519 72.793864) (width 0.2) (layer "F.Cu") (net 18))
 (segment (start 156.385 93.65) (end 158.819519 91.215481) (width 0.2) (layer "F.Cu") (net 18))
 (segment (start 117.24 85.470972) (end 119.557977 83.152995) (width 0.2) (layer "F.Cu") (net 3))
 (segment (start 117.24 89.84) (end 117.24 85.470972) (width 0.2) (layer "F.Cu") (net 3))
 (segment (start 155.235489 95.040489) (end 156.620166 95.040489) (width 0.2) (layer "F.Cu") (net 5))
 (segment (start 156.620166 95.040489) (end 158.819518 92.841137) (width 0.2) (layer "F.Cu") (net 5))
 (segment (start 150.425498 99.85048) (end 155.235489 95.040489) (width 0.2) (layer "F.Cu") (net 5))
 (segment (start 128.072693 99.85048) (end 150.425498 99.85048) (width 0.2) (layer "F.Cu") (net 5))
 (segment (start 119.24 91.017787) (end 128.072693 99.85048) (width 0.2) (layer "F.Cu") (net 5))
 (segment (start 158.819518 92.841137) (end 158.819518 91.780488) (width 0.2) (layer "F.Cu") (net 5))
 (segment (start 119.24 89.84) (end 119.24 91.017787) (width 0.2) (layer "F.Cu") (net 5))
 (segment (start 118.24 89.84) (end 118.24 85.035978) (width 0.2) (layer "F.Cu") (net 4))
 (segment (start 118.24 85.035978) (end 119.84048 83.435498) (width 0.2) (layer "F.Cu") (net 4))
 (segment (start 99.85048 111.73048) (end 99.85048 80.42) (width 0.2) (layer "F.Cu") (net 10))
 (segment (start 153.34 82.985) (end 153.34 77.14) (width 0.2) (layer "F.Cu") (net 10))
 (segment (start 108.255 80.42) (end 108.255 74.885) (width 0.2) (layer "F.Cu") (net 10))
 (segment (start 99.85048 111.73048) (end 99.85048 79.68) (width 0.2) (layer "F.Cu") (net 10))
 (segment (start 108.255 74.885) (end 108.37 74.77) (width 0.2) (layer "F.Cu") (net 10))
 (segment (start 107.17 119.05) (end 99.85048 111.73048) (width 0.2) (layer "F.Cu") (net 10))
 (segment (start 156.385 86.03) (end 153.34 82.985) (width 0.2) (layer "F.Cu") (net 10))
 (segment (start 153.34 77.14) (end 131.06 77.14) (width 0.2) (layer "F.Cu") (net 10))
 (segment (start 131.06 77.14) (end 128.69 74.77) (width 0.2) (layer "F.Cu") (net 10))
 (segment (start 99.45096 112.929982) (end 99.45096 72.091212) (width 0.2) (layer "F.Cu") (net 11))
 (segment (start 99.45096 72.091212) (end 101.691692 69.85048) (width 0.2) (layer "F.Cu") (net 11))
 (segment (start 108.910489 119.849511) (end 106.370489 119.849511) (width 0.2) (layer "F.Cu") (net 11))
 (segment (start 101.691692 69.85048) (end 112.065 69.85048) (width 0.2) (layer "F.Cu") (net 11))
 (segment (start 109.71 119.05) (end 108.910489 119.849511) (width 0.2) (layer "F.Cu") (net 11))
 (segment (start 106.370489 119.849511) (end 99.45096 112.929982) (width 0.2) (layer "F.Cu") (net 11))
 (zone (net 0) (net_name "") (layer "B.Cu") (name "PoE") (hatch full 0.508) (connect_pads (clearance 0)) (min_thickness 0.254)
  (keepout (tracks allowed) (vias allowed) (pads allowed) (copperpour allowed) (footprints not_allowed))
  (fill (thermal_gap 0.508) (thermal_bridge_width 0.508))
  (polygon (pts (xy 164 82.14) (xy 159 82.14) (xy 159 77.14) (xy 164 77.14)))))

